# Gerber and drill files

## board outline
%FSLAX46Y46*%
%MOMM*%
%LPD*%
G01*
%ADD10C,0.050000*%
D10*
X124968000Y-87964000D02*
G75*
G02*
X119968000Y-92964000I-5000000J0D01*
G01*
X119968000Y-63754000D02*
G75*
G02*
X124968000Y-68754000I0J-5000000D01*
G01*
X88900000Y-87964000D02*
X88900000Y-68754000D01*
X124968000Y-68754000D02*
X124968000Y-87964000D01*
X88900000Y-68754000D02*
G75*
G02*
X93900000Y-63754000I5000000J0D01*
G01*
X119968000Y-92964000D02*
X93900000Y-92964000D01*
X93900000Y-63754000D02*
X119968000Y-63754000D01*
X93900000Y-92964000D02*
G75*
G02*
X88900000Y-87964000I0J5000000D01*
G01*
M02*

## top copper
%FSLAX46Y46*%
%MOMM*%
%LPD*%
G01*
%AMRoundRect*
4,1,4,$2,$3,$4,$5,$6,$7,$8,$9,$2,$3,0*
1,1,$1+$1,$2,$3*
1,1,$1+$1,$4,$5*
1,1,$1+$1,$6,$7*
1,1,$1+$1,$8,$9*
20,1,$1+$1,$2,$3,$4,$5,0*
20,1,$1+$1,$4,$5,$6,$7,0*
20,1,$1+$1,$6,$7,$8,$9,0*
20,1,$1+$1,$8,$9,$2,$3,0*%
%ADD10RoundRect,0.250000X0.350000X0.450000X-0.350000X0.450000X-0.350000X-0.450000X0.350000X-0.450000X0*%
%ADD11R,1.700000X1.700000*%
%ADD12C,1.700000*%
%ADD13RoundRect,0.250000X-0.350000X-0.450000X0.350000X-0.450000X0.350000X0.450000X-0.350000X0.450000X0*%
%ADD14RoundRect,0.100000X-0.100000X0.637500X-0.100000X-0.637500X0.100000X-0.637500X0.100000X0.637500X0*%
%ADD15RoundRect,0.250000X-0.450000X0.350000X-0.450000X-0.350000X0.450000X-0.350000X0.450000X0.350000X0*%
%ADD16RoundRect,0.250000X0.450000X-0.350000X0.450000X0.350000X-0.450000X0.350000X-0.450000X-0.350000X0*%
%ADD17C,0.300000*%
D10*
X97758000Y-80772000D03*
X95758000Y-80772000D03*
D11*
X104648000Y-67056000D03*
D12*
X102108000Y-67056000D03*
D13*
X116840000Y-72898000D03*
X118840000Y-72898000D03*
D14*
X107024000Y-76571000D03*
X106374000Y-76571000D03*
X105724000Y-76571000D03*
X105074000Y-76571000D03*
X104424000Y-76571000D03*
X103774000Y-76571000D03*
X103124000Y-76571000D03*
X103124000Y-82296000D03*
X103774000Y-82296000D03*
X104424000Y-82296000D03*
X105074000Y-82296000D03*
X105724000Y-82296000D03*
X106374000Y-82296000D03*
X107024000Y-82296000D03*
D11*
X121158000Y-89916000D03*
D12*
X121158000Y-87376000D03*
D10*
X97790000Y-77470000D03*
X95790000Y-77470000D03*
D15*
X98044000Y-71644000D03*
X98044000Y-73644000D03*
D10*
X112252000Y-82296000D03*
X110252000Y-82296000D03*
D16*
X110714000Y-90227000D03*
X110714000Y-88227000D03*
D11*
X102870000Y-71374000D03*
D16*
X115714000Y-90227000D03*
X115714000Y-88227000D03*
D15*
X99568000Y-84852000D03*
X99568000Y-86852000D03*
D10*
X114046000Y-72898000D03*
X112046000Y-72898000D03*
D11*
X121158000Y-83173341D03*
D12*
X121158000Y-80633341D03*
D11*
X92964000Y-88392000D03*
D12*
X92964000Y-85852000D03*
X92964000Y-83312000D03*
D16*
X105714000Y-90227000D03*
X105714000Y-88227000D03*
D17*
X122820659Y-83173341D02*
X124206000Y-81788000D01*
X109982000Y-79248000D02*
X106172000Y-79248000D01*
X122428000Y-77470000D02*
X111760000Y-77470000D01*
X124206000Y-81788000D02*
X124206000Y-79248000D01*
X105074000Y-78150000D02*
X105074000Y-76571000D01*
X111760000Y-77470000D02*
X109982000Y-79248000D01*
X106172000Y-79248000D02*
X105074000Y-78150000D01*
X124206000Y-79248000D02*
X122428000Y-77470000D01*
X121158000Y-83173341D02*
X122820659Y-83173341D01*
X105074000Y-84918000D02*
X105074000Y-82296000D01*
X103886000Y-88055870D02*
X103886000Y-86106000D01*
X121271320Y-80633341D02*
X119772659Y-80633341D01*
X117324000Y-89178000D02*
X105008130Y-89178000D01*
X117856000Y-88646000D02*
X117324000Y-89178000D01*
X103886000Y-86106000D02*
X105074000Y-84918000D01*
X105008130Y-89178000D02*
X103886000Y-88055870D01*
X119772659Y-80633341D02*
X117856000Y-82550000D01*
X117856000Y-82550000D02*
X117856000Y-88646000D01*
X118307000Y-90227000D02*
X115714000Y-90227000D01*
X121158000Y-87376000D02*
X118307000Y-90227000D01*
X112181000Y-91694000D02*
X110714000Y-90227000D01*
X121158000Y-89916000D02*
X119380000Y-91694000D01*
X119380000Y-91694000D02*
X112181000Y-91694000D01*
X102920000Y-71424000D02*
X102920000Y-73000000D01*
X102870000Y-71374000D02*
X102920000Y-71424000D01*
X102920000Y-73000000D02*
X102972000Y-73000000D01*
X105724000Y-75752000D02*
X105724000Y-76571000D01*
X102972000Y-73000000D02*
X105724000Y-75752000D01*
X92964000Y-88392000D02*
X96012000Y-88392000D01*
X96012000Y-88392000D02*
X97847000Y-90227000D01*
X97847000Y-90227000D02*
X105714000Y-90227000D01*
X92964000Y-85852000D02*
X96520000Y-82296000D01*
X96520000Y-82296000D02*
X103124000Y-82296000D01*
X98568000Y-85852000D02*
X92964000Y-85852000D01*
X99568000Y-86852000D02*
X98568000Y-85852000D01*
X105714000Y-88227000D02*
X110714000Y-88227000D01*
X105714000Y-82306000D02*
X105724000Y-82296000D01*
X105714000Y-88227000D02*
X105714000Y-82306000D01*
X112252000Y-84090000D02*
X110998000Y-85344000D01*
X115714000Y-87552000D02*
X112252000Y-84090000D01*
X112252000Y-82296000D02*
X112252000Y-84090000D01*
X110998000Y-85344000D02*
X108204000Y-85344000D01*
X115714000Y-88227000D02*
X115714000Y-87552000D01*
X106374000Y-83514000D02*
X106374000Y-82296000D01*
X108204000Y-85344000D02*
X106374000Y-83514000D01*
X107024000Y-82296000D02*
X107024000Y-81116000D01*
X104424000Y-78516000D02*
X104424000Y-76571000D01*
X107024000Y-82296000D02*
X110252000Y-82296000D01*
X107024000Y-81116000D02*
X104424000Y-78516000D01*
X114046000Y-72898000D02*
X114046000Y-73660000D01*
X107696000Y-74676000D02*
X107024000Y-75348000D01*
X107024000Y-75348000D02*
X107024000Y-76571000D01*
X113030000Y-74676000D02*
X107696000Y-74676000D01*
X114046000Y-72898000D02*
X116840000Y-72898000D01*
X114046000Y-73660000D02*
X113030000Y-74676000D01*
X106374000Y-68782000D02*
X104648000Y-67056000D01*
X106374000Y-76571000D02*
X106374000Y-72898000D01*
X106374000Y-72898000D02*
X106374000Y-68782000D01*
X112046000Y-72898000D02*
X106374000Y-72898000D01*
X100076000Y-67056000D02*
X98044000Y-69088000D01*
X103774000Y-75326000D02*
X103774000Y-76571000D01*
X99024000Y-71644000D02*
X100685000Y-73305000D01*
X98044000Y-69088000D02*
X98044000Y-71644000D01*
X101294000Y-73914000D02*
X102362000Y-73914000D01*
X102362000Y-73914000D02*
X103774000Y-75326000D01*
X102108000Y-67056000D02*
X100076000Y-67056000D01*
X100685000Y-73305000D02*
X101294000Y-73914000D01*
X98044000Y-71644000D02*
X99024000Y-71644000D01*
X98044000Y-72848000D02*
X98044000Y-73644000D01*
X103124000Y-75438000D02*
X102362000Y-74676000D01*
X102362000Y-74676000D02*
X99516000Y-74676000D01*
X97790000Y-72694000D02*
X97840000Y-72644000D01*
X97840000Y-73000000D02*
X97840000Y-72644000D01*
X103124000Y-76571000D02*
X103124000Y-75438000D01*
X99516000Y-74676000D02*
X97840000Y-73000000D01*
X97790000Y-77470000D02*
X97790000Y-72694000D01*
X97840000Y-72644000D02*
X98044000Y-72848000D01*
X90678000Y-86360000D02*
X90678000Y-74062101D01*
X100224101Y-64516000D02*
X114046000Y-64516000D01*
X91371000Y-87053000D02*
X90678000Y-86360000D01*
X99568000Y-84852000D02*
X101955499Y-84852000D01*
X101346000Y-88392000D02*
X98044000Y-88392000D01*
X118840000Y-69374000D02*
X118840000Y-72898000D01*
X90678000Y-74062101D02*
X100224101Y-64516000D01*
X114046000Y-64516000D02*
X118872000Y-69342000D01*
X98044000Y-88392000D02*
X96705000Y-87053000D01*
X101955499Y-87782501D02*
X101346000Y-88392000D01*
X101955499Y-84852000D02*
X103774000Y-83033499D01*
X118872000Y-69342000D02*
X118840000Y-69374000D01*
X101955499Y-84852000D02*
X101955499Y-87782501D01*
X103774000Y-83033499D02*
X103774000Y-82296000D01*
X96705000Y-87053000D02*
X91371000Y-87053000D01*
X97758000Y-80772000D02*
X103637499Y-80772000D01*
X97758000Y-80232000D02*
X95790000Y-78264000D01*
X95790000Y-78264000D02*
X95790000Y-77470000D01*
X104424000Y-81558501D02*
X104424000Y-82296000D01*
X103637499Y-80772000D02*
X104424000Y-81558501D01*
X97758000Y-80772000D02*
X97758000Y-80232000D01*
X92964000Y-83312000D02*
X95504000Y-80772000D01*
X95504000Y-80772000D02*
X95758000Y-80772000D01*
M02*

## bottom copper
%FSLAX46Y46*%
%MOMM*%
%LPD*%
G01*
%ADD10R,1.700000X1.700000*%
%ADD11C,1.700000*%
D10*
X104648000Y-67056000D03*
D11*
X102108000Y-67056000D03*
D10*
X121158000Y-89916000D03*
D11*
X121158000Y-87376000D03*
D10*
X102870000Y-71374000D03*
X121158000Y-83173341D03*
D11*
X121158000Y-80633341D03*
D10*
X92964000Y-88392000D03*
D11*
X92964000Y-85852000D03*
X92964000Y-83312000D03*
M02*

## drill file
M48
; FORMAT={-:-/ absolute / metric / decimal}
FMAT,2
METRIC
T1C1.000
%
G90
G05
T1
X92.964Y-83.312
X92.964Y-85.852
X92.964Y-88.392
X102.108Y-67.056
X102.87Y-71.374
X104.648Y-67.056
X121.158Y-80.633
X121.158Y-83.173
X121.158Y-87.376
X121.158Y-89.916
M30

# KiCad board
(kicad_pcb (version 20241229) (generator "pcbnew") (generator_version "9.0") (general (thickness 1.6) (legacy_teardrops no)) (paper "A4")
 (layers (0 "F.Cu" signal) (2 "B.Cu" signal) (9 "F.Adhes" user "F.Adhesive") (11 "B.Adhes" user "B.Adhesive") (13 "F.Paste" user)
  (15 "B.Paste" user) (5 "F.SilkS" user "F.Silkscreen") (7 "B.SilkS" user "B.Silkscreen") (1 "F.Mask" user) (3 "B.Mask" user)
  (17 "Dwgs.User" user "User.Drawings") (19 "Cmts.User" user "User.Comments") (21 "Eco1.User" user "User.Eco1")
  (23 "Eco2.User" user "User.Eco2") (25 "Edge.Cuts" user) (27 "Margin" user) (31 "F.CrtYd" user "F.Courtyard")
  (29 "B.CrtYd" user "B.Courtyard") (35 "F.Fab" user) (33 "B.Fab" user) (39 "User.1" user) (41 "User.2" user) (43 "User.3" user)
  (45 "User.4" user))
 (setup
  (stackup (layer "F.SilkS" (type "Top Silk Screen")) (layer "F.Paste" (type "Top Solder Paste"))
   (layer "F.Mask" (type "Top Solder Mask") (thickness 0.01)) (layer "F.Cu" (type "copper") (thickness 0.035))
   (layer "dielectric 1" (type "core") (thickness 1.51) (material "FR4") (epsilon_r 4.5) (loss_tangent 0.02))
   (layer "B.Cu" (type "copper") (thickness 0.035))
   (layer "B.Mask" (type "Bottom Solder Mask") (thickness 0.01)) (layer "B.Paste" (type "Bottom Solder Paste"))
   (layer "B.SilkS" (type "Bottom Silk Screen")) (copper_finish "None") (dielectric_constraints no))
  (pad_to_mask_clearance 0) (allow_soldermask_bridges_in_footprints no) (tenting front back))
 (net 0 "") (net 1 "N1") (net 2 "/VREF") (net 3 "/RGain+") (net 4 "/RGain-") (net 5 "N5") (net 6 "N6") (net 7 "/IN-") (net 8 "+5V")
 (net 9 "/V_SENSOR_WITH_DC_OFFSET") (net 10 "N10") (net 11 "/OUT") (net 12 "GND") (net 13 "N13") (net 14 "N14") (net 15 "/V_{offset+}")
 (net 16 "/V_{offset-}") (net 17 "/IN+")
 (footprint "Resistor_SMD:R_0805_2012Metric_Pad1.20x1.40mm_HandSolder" (layer "F.Cu") (at 96.758 80.772 180)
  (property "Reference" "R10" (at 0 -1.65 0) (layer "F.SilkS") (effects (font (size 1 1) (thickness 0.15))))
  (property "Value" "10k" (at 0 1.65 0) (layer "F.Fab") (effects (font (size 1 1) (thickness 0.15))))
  (pad "1" smd roundrect (at -1 0 180) (size 1.2 1.4) (layers "F.Cu" "F.Mask" "F.Paste") (roundrect_rratio 0.208333) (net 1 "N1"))
  (pad "2" smd roundrect (at 1 0 180) (size 1.2 1.4) (layers "F.Cu" "F.Mask" "F.Paste") (roundrect_rratio 0.208333) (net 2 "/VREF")))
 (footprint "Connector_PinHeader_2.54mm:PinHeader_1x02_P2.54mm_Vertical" (layer "F.Cu") (at 104.648 67.056 -90)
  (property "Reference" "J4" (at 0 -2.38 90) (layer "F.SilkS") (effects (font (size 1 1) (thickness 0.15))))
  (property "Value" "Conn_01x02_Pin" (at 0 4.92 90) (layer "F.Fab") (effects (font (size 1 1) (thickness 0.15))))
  (pad "1" thru_hole rect (at 0 0 270) (size 1.7 1.7) (drill 1) (layers "*.Cu" "*.Mask") (remove_unused_layers no) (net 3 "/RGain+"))
  (pad "2" thru_hole circle (at 0 2.54 270) (size 1.7 1.7) (drill 1) (layers "*.Cu" "*.Mask") (remove_unused_layers no) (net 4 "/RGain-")))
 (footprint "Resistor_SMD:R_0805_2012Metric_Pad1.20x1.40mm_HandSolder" (layer "F.Cu") (at 117.84 72.898)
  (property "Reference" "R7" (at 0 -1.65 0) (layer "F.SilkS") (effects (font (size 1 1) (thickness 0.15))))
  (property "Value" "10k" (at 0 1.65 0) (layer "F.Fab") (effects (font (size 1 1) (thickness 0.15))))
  (pad "1" smd roundrect (at -1 0) (size 1.2 1.4) (layers "F.Cu" "F.Mask" "F.Paste") (roundrect_rratio 0.208333) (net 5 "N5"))
  (pad "2" smd roundrect (at 1 0) (size 1.2 1.4) (layers "F.Cu" "F.Mask" "F.Paste") (roundrect_rratio 0.208333) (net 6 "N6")))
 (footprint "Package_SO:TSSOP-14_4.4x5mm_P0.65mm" (layer "F.Cu") (at 105.074 79.4335 -90)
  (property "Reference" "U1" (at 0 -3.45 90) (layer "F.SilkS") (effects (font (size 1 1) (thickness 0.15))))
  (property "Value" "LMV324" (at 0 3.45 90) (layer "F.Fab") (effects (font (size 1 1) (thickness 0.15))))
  (pad "1" smd roundrect (at -2.8625 -1.95 270) (size 1.475 0.4) (layers "F.Cu" "F.Mask" "F.Paste") (roundrect_rratio 0.25) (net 5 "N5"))
  (pad "2" smd roundrect (at -2.8625 -1.3 270) (size 1.475 0.4) (layers "F.Cu" "F.Mask" "F.Paste") (roundrect_rratio 0.25) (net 3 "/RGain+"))
  (pad "3" smd roundrect (at -2.8625 -0.65 270) (size 1.475 0.4) (layers "F.Cu" "F.Mask" "F.Paste") (roundrect_rratio 0.25) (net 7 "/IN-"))
  (pad "4" smd roundrect (at -2.8625 0 270) (size 1.475 0.4) (layers "F.Cu" "F.Mask" "F.Paste") (roundrect_rratio 0.25) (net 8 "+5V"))
  (pad "5" smd roundrect (at -2.8625 0.65 270) (size 1.475 0.4) (layers "F.Cu" "F.Mask" "F.Paste") (roundrect_rratio 0.25)
   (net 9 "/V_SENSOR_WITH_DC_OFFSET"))
  (pad "6" smd roundrect (at -2.8625 1.3 270) (size 1.475 0.4) (layers "F.Cu" "F.Mask" "F.Paste") (roundrect_rratio 0.25) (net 4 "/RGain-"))
  (pad "7" smd roundrect (at -2.8625 1.95 270) (size 1.475 0.4) (layers "F.Cu" "F.Mask" "F.Paste") (roundrect_rratio 0.25) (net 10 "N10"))
  (pad "8" smd roundrect (at 2.8625 1.95 270) (size 1.475 0.4) (layers "F.Cu" "F.Mask" "F.Paste") (roundrect_rratio 0.25) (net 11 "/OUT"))
  (pad "9" smd roundrect (at 2.8625 1.3 270) (size 1.475 0.4) (layers "F.Cu" "F.Mask" "F.Paste") (roundrect_rratio 0.25) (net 6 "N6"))
  (pad "10" smd roundrect (at 2.8625 0.65 270) (size 1.475 0.4) (layers "F.Cu" "F.Mask" "F.Paste") (roundrect_rratio 0.25) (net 1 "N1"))
  (pad "11" smd roundrect (at 2.8625 0 270) (size 1.475 0.4) (layers "F.Cu" "F.Mask" "F.Paste") (roundrect_rratio 0.25) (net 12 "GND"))
  (pad "12" smd roundrect (at 2.8625 -0.65 270) (size 1.475 0.4) (layers "F.Cu" "F.Mask" "F.Paste") (roundrect_rratio 0.25) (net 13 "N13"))
  (pad "13" smd roundrect (at 2.8625 -1.3 270) (size 1.475 0.4) (layers "F.Cu" "F.Mask" "F.Paste") (roundrect_rratio 0.25) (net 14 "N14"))
  (pad "14" smd roundrect (at 2.8625 -1.95 270) (size 1.475 0.4) (layers "F.Cu" "F.Mask" "F.Paste") (roundrect_rratio 0.25)
   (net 9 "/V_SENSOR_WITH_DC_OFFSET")))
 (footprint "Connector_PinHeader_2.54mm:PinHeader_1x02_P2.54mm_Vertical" (layer "F.Cu") (at 121.158 89.916 180)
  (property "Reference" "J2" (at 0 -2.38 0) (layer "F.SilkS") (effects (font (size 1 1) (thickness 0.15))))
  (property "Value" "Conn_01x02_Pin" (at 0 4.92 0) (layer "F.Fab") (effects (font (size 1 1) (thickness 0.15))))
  (pad "1" thru_hole rect (at 0 0 180) (size 1.7 1.7) (drill 1) (layers "*.Cu" "*.Mask") (remove_unused_layers no) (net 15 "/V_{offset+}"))
  (pad "2" thru_hole circle (at 0 2.54 180) (size 1.7 1.7) (drill 1) (layers "*.Cu" "*.Mask") (remove_unused_layers no)
   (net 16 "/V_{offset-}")))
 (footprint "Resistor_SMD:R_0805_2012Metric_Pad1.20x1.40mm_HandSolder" (layer "F.Cu") (at 96.79 77.47 180)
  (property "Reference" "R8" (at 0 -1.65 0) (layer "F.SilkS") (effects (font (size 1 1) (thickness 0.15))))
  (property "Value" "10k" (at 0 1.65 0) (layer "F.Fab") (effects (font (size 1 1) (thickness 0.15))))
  (pad "1" smd roundrect (at -1 0 180) (size 1.2 1.4) (layers "F.Cu" "F.Mask" "F.Paste") (roundrect_rratio 0.208333) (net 10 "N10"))
  (pad "2" smd roundrect (at 1 0 180) (size 1.2 1.4) (layers "F.Cu" "F.Mask" "F.Paste") (roundrect_rratio 0.208333) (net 1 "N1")))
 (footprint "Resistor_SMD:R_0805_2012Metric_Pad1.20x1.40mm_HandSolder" (layer "F.Cu") (at 98.044 72.644 -90)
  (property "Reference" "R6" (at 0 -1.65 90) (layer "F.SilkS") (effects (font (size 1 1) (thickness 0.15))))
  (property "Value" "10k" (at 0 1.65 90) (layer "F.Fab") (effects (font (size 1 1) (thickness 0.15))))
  (pad "1" smd roundrect (at -1 0 270) (size 1.2 1.4) (layers "F.Cu" "F.Mask" "F.Paste") (roundrect_rratio 0.208333) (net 4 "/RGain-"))
  (pad "2" smd roundrect (at 1 0 270) (size 1.2 1.4) (layers "F.Cu" "F.Mask" "F.Paste") (roundrect_rratio 0.208333) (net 10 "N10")))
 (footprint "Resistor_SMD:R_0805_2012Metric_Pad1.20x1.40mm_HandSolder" (layer "F.Cu") (at 111.252 82.296 180)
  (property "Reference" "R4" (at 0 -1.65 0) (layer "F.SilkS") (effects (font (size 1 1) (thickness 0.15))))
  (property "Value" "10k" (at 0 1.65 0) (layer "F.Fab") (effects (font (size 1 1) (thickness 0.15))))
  (pad "1" smd roundrect (at -1 0 180) (size 1.2 1.4) (layers "F.Cu" "F.Mask" "F.Paste") (roundrect_rratio 0.208333) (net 14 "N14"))
  (pad "2" smd roundrect (at 1 0 180) (size 1.2 1.4) (layers "F.Cu" "F.Mask" "F.Paste") (roundrect_rratio 0.208333)
   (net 9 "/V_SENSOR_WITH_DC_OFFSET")))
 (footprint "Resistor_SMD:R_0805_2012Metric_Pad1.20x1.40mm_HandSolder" (layer "F.Cu") (at 110.714 89.227 90)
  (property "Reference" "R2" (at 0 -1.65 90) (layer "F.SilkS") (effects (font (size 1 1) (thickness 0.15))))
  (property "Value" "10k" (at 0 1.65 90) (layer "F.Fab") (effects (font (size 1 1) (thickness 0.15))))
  (pad "1" smd roundrect (at -1 0 90) (size 1.2 1.4) (layers "F.Cu" "F.Mask" "F.Paste") (roundrect_rratio 0.208333) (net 15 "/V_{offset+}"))
  (pad "2" smd roundrect (at 1 0 90) (size 1.2 1.4) (layers "F.Cu" "F.Mask" "F.Paste") (roundrect_rratio 0.208333) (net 13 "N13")))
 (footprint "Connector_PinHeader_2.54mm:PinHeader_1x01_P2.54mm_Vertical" (layer "F.Cu") (at 102.87 71.374)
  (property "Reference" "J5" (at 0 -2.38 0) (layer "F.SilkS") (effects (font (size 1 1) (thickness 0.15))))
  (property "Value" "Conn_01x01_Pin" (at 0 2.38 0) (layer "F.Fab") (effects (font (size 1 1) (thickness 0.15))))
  (pad "1" thru_hole rect (at 0 0) (size 1.7 1.7) (drill 1) (layers "*.Cu" "*.Mask") (remove_unused_layers no) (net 7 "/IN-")))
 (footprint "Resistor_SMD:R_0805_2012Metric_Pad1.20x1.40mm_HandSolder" (layer "F.Cu") (at 115.714 89.227 90)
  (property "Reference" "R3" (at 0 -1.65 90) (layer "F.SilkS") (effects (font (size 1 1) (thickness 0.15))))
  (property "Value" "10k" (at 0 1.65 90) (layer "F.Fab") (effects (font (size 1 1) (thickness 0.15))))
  (pad "1" smd roundrect (at -1 0 90) (size 1.2 1.4) (layers "F.Cu" "F.Mask" "F.Paste") (roundrect_rratio 0.208333) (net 16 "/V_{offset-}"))
  (pad "2" smd roundrect (at 1 0 90) (size 1.2 1.4) (layers "F.Cu" "F.Mask" "F.Paste") (roundrect_rratio 0.208333) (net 14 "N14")))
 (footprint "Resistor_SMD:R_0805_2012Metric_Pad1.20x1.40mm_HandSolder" (layer "F.Cu") (at 99.568 85.852 -90)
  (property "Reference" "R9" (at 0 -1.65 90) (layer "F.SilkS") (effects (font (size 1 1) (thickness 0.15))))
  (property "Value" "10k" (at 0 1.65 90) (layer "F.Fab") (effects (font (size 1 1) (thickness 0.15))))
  (pad "1" smd roundrect (at -1 0 270) (size 1.2 1.4) (layers "F.Cu" "F.Mask" "F.Paste") (roundrect_rratio 0.208333) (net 6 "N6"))
  (pad "2" smd roundrect (at 1 0 270) (size 1.2 1.4) (layers "F.Cu" "F.Mask" "F.Paste") (roundrect_rratio 0.208333) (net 11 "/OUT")))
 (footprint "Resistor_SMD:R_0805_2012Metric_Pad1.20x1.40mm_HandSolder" (layer "F.Cu") (at 113.046 72.898 180)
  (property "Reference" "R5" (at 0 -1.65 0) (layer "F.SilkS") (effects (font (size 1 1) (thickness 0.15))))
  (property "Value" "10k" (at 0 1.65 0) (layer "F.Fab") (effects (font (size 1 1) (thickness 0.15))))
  (pad "1" smd roundrect (at -1 0 180) (size 1.2 1.4) (layers "F.Cu" "F.Mask" "F.Paste") (roundrect_rratio 0.208333) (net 5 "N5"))
  (pad "2" smd roundrect (at 1 0 180) (size 1.2 1.4) (layers "F.Cu" "F.Mask" "F.Paste") (roundrect_rratio 0.208333) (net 3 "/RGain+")))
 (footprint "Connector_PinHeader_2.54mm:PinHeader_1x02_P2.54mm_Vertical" (layer "F.Cu") (at 121.158 83.173341 180)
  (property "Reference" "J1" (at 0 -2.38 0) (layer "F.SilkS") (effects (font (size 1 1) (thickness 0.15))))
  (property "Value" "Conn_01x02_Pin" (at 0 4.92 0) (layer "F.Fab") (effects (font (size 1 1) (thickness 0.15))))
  (pad "1" thru_hole rect (at 0 0 180) (size 1.7 1.7) (drill 1) (layers "*.Cu" "*.Mask") (remove_unused_layers no) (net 8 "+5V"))
  (pad "2" thru_hole circle (at 0 2.54 180) (size 1.7 1.7) (drill 1) (layers "*.Cu" "*.Mask") (remove_unused_layers no) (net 12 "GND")))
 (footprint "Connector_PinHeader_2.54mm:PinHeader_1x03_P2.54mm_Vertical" (layer "F.Cu") (at 92.964 88.392 180)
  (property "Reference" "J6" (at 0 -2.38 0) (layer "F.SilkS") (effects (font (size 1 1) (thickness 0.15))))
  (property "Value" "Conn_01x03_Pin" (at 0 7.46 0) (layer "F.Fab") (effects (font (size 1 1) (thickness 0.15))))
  (pad "1" thru_hole rect (at 0 0 180) (size 1.7 1.7) (drill 1) (layers "*.Cu" "*.Mask") (remove_unused_layers no) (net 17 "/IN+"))
  (pad "2" thru_hole circle (at 0 2.54 180) (size 1.7 1.7) (drill 1) (layers "*.Cu" "*.Mask") (remove_unused_layers no) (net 11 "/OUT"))
  (pad "3" thru_hole circle (at 0 5.08 180) (size 1.7 1.7) (drill 1) (layers "*.Cu" "*.Mask") (remove_unused_layers no) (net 2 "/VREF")))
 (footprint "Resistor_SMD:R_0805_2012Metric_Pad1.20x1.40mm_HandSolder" (layer "F.Cu") (at 105.714 89.227 90)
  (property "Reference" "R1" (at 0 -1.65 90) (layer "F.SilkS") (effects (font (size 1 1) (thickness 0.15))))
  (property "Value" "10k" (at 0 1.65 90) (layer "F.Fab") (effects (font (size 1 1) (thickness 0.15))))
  (pad "1" smd roundrect (at -1 0 90) (size 1.2 1.4) (layers "F.Cu" "F.Mask" "F.Paste") (roundrect_rratio 0.208333) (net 17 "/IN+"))
  (pad "2" smd roundrect (at 1 0 90) (size 1.2 1.4) (layers "F.Cu" "F.Mask" "F.Paste") (roundrect_rratio 0.208333) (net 13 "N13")))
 (gr_arc (start 124.968 87.964) (mid 123.503534 91.499534) (end 119.968 92.964) (stroke (width 0.05) (type default)) (layer "Edge.Cuts"))
 (gr_arc (start 119.968 63.754) (mid 123.503534 65.218466) (end 124.968 68.754) (stroke (width 0.05) (type default)) (layer "Edge.Cuts"))
 (gr_line (start 88.9 87.964) (end 88.9 68.754) (stroke (width 0.05) (type default)) (layer "Edge.Cuts"))
 (gr_line (start 124.968 68.754) (end 124.968 87.964) (stroke (width 0.05) (type default)) (layer "Edge.Cuts"))
 (gr_arc (start 88.9 68.754) (mid 90.364466 65.218466) (end 93.9 63.754) (stroke (width 0.05) (type default)) (layer "Edge.Cuts"))
 (gr_line (start 119.968 92.964) (end 93.9 92.964) (stroke (width 0.05) (type default)) (layer "Edge.Cuts"))
 (gr_line (start 93.9 63.754) (end 119.968 63.754) (stroke (width 0.05) (type default)) (layer "Edge.Cuts"))
 (gr_arc (start 93.9 92.964) (mid 90.364466 91.499534) (end 88.9 87.964) (stroke (width 0.05) (type default)) (layer "Edge.Cuts"))
 (segment (start 122.820659 83.173341) (end 124.206 81.788) (width 0.3) (layer "F.Cu") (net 8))
 (segment (start 109.982 79.248) (end 106.172 79.248) (width 0.3) (layer "F.Cu") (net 8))
 (segment (start 122.428 77.47) (end 111.76 77.47) (width 0.3) (layer "F.Cu") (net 8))
 (segment (start 124.206 81.788) (end 124.206 79.248) (width 0.3) (layer "F.Cu") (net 8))
 (segment (start 105.074 78.15) (end 105.074 76.571) (width 0.3) (layer "F.Cu") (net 8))
 (segment (start 111.76 77.47) (end 109.982 79.248) (width 0.3) (layer "F.Cu") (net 8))
 (segment (start 106.172 79.248) (end 105.074 78.15) (width 0.3) (layer "F.Cu") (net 8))
 (segment (start 124.206 79.248) (end 122.428 77.47) (width 0.3) (layer "F.Cu") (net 8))
 (segment (start 121.158 83.173341) (end 122.820659 83.173341) (width 0.3) (layer "F.Cu") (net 8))
 (segment (start 105.074 84.918) (end 105.074 82.296) (width 0.3) (layer "F.Cu") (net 12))
 (segment (start 103.886 88.05587) (end 103.886 86.106) (width 0.3) (layer "F.Cu") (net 12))
 (segment (start 121.27132 80.633341) (end 119.772659 80.633341) (width 0.3) (layer "F.Cu") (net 12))
 (segment (start 117.324 89.178) (end 105.00813 89.178) (width 0.3) (layer "F.Cu") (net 12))
 (segment (start 117.856 88.646) (end 117.324 89.178) (width 0.3) (layer "F.Cu") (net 12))
 (segment (start 103.886 86.106) (end 105.074 84.918) (width 0.3) (layer "F.Cu") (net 12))
 (segment (start 105.00813 89.178) (end 103.886 88.05587) (width 0.3) (layer "F.Cu") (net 12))
 (segment (start 119.772659 80.633341) (end 117.856 82.55) (width 0.3) (layer "F.Cu") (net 12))
 (segment (start 117.856 82.55) (end 117.856 88.646) (width 0.3) (layer "F.Cu") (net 12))
 (segment (start 118.307 90.227) (end 115.714 90.227) (width 0.3) (layer "F.Cu") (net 16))
 (segment (start 121.158 87.376) (end 118.307 90.227) (width 0.3) (layer "F.Cu") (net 16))
 (segment (start 112.181 91.694) (end 110.714 90.227) (width 0.3) (layer "F.Cu") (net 15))
 (segment (start 121.158 89.916) (end 119.38 91.694) (width 0.3) (layer "F.Cu") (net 15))
 (segment (start 119.38 91.694) (end 112.181 91.694) (width 0.3) (layer "F.Cu") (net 15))
 (segment (start 102.92 71.424) (end 102.92 73) (width 0.3) (layer "F.Cu") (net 7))
 (segment (start 102.87 71.374) (end 102.92 71.424) (width 0.3) (layer "F.Cu") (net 7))
 (segment (start 102.92 73) (end 102.972 73) (width 0.3) (layer "F.Cu") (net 7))
 (segment (start 105.724 75.752) (end 105.724 76.571) (width 0.3) (layer "F.Cu") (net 7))
 (segment (start 102.972 73) (end 105.724 75.752) (width 0.3) (layer "F.Cu") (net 7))
 (segment (start 92.964 88.392) (end 96.012 88.392) (width 0.3) (layer "F.Cu") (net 17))
 (segment (start 96.012 88.392) (end 97.847 90.227) (width 0.3) (layer "F.Cu") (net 17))
 (segment (start 97.847 90.227) (end 105.714 90.227) (width 0.3) (layer "F.Cu") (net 17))
 (segment (start 92.964 85.852) (end 96.52 82.296) (width 0.3) (layer "F.Cu") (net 11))
 (segment (start 96.52 82.296) (end 103.124 82.296) (width 0.3) (layer "F.Cu") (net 11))
 (segment (start 98.568 85.852) (end 92.964 85.852) (width 0.3) (layer "F.Cu") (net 11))
 (segment (start 99.568 86.852) (end 98.568 85.852) (width 0.3) (layer "F.Cu") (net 11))
 (segment (start 105.714 88.227) (end 110.714 88.227) (width 0.3) (layer "F.Cu") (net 13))
 (segment (start 105.714 82.306) (end 105.724 82.296) (width 0.3) (layer "F.Cu") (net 13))
 (segment (start 105.714 88.227) (end 105.714 82.306) (width 0.3) (layer "F.Cu") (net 13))
 (segment (start 112.252 84.09) (end 110.998 85.344) (width 0.3) (layer "F.Cu") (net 14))
 (segment (start 115.714 87.552) (end 112.252 84.09) (width 0.3) (layer "F.Cu") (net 14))
 (segment (start 112.252 82.296) (end 112.252 84.09) (width 0.3) (layer "F.Cu") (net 14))
 (segment (start 110.998 85.344) (end 108.204 85.344) (width 0.3) (layer "F.Cu") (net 14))
 (segment (start 115.714 88.227) (end 115.714 87.552) (width 0.3) (layer "F.Cu") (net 14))
 (segment (start 106.374 83.514) (end 106.374 82.296) (width 0.3) (layer "F.Cu") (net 14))
 (segment (start 108.204 85.344) (end 106.374 83.514) (width 0.3) (layer "F.Cu") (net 14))
 (segment (start 107.024 82.296) (end 107.024 81.116) (width 0.3) (layer "F.Cu") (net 9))
 (segment (start 104.424 78.516) (end 104.424 76.571) (width 0.3) (layer "F.Cu") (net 9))
 (segment (start 107.024 82.296) (end 110.252 82.296) (width 0.3) (layer "F.Cu") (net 9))
 (segment (start 107.024 81.116) (end 104.424 78.516) (width 0.3) (layer "F.Cu") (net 9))
 (segment (start 114.046 72.898) (end 114.046 73.66) (width 0.3) (layer "F.Cu") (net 5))
 (segment (start 107.696 74.676) (end 107.024 75.348) (width 0.3) (layer "F.Cu") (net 5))
 (segment (start 107.024 75.348) (end 107.024 76.571) (width 0.3) (layer "F.Cu") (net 5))
 (segment (start 113.03 74.676) (end 107.696 74.676) (width 0.3) (layer "F.Cu") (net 5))
 (segment (start 114.046 72.898) (end 116.84 72.898) (width 0.3) (layer "F.Cu") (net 5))
 (segment (start 114.046 73.66) (end 113.03 74.676) (width 0.3) (layer "F.Cu") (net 5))
 (segment (start 106.374 68.782) (end 104.648 67.056) (width 0.3) (layer "F.Cu") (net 3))
 (segment (start 106.374 76.571) (end 106.374 72.898) (width 0.3) (layer "F.Cu") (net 3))
 (segment (start 106.374 72.898) (end 106.374 68.782) (width 0.3) (layer "F.Cu") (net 3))
 (segment (start 112.046 72.898) (end 106.374 72.898) (width 0.3) (layer "F.Cu") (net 3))
 (segment (start 100.076 67.056) (end 98.044 69.088) (width 0.3) (layer "F.Cu") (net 4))
 (segment (start 103.774 75.326) (end 103.774 76.571) (width 0.3) (layer "F.Cu") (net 4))
 (segment (start 99.024 71.644) (end 100.685 73.305) (width 0.3) (layer "F.Cu") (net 4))
 (segment (start 98.044 69.088) (end 98.044 71.644) (width 0.3) (layer "F.Cu") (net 4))
 (segment (start 101.294 73.914) (end 102.362 73.914) (width 0.3) (layer "F.Cu") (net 4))
 (segment (start 102.362 73.914) (end 103.774 75.326) (width 0.3) (layer "F.Cu") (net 4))
 (segment (start 102.108 67.056) (end 100.076 67.056) (width 0.3) (layer "F.Cu") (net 4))
 (segment (start 100.685 73.305) (end 101.294 73.914) (width 0.3) (layer "F.Cu") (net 4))
 (segment (start 98.044 71.644) (end 99.024 71.644) (width 0.3) (layer "F.Cu") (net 4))
 (segment (start 98.044 72.848) (end 98.044 73.644) (width 0.3) (layer "F.Cu") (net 10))
 (segment (start 103.124 75.438) (end 102.362 74.676) (width 0.3) (layer "F.Cu") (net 10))
 (segment (start 102.362 74.676) (end 99.516 74.676) (width 0.3) (layer "F.Cu") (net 10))
 (segment (start 97.79 72.694) (end 97.84 72.644) (width 0.3) (layer "F.Cu") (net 10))
 (segment (start 97.84 73) (end 97.84 72.644) (width 0.3) (layer "F.Cu") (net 10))
 (segment (start 103.124 76.571) (end 103.124 75.438) (width 0.3) (layer "F.Cu") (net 10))
 (segment (start 99.516 74.676) (end 97.84 73) (width 0.3) (layer "F.Cu") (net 10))
 (segment (start 97.79 77.47) (end 97.79 72.694) (width 0.3) (layer "F.Cu") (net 10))
 (segment (start 97.84 72.644) (end 98.044 72.848) (width 0.3) (layer "F.Cu") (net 10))
 (segment (start 90.678 86.36) (end 90.678 74.062101) (width 0.3) (layer "F.Cu") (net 6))
 (segment (start 100.224101 64.516) (end 114.046 64.516) (width 0.3) (layer "F.Cu") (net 6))
 (segment (start 91.371 87.053) (end 90.678 86.36) (width 0.3) (layer "F.Cu") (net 6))
 (segment (start 99.568 84.852) (end 101.955499 84.852) (width 0.3) (layer "F.Cu") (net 6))
 (segment (start 101.346 88.392) (end 98.044 88.392) (width 0.3) (layer "F.Cu") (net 6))
 (segment (start 118.84 69.374) (end 118.84 72.898) (width 0.3) (layer "F.Cu") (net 6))
 (segment (start 90.678 74.062101) (end 100.224101 64.516) (width 0.3) (layer "F.Cu") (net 6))
 (segment (start 114.046 64.516) (end 118.872 69.342) (width 0.3) (layer "F.Cu") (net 6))
 (segment (start 98.044 88.392) (end 96.705 87.053) (width 0.3) (layer "F.Cu") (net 6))
 (segment (start 101.955499 87.782501) (end 101.346 88.392) (width 0.3) (layer "F.Cu") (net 6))
 (segment (start 101.955499 84.852) (end 103.774 83.033499) (width 0.3) (layer "F.Cu") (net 6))
 (segment (start 118.872 69.342) (end 118.84 69.374) (width 0.3) (layer "F.Cu") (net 6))
 (segment (start 101.955499 84.852) (end 101.955499 87.782501) (width 0.3) (layer "F.Cu") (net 6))
 (segment (start 103.774 83.033499) (end 103.774 82.296) (width 0.3) (layer "F.Cu") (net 6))
 (segment (start 96.705 87.053) (end 91.371 87.053) (width 0.3) (layer "F.Cu") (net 6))
 (segment (start 97.758 80.772) (end 103.637499 80.772) (width 0.3) (layer "F.Cu") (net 1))
 (segment (start 97.758 80.232) (end 95.79 78.264) (width 0.3) (layer "F.Cu") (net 1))
 (segment (start 95.79 78.264) (end 95.79 77.47) (width 0.3) (layer "F.Cu") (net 1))
 (segment (start 104.424 81.558501) (end 104.424 82.296) (width 0.3) (layer "F.Cu") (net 1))
 (segment (start 103.637499 80.772) (end 104.424 81.558501) (width 0.3) (layer "F.Cu") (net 1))
 (segment (start 97.758 80.772) (end 97.758 80.232) (width 0.3) (layer "F.Cu") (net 1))
 (segment (start 92.964 83.312) (end 95.504 80.772) (width 0.3) (layer "F.Cu") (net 2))
 (segment (start 95.504 80.772) (end 95.758 80.772) (width 0.3) (layer "F.Cu") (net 2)))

